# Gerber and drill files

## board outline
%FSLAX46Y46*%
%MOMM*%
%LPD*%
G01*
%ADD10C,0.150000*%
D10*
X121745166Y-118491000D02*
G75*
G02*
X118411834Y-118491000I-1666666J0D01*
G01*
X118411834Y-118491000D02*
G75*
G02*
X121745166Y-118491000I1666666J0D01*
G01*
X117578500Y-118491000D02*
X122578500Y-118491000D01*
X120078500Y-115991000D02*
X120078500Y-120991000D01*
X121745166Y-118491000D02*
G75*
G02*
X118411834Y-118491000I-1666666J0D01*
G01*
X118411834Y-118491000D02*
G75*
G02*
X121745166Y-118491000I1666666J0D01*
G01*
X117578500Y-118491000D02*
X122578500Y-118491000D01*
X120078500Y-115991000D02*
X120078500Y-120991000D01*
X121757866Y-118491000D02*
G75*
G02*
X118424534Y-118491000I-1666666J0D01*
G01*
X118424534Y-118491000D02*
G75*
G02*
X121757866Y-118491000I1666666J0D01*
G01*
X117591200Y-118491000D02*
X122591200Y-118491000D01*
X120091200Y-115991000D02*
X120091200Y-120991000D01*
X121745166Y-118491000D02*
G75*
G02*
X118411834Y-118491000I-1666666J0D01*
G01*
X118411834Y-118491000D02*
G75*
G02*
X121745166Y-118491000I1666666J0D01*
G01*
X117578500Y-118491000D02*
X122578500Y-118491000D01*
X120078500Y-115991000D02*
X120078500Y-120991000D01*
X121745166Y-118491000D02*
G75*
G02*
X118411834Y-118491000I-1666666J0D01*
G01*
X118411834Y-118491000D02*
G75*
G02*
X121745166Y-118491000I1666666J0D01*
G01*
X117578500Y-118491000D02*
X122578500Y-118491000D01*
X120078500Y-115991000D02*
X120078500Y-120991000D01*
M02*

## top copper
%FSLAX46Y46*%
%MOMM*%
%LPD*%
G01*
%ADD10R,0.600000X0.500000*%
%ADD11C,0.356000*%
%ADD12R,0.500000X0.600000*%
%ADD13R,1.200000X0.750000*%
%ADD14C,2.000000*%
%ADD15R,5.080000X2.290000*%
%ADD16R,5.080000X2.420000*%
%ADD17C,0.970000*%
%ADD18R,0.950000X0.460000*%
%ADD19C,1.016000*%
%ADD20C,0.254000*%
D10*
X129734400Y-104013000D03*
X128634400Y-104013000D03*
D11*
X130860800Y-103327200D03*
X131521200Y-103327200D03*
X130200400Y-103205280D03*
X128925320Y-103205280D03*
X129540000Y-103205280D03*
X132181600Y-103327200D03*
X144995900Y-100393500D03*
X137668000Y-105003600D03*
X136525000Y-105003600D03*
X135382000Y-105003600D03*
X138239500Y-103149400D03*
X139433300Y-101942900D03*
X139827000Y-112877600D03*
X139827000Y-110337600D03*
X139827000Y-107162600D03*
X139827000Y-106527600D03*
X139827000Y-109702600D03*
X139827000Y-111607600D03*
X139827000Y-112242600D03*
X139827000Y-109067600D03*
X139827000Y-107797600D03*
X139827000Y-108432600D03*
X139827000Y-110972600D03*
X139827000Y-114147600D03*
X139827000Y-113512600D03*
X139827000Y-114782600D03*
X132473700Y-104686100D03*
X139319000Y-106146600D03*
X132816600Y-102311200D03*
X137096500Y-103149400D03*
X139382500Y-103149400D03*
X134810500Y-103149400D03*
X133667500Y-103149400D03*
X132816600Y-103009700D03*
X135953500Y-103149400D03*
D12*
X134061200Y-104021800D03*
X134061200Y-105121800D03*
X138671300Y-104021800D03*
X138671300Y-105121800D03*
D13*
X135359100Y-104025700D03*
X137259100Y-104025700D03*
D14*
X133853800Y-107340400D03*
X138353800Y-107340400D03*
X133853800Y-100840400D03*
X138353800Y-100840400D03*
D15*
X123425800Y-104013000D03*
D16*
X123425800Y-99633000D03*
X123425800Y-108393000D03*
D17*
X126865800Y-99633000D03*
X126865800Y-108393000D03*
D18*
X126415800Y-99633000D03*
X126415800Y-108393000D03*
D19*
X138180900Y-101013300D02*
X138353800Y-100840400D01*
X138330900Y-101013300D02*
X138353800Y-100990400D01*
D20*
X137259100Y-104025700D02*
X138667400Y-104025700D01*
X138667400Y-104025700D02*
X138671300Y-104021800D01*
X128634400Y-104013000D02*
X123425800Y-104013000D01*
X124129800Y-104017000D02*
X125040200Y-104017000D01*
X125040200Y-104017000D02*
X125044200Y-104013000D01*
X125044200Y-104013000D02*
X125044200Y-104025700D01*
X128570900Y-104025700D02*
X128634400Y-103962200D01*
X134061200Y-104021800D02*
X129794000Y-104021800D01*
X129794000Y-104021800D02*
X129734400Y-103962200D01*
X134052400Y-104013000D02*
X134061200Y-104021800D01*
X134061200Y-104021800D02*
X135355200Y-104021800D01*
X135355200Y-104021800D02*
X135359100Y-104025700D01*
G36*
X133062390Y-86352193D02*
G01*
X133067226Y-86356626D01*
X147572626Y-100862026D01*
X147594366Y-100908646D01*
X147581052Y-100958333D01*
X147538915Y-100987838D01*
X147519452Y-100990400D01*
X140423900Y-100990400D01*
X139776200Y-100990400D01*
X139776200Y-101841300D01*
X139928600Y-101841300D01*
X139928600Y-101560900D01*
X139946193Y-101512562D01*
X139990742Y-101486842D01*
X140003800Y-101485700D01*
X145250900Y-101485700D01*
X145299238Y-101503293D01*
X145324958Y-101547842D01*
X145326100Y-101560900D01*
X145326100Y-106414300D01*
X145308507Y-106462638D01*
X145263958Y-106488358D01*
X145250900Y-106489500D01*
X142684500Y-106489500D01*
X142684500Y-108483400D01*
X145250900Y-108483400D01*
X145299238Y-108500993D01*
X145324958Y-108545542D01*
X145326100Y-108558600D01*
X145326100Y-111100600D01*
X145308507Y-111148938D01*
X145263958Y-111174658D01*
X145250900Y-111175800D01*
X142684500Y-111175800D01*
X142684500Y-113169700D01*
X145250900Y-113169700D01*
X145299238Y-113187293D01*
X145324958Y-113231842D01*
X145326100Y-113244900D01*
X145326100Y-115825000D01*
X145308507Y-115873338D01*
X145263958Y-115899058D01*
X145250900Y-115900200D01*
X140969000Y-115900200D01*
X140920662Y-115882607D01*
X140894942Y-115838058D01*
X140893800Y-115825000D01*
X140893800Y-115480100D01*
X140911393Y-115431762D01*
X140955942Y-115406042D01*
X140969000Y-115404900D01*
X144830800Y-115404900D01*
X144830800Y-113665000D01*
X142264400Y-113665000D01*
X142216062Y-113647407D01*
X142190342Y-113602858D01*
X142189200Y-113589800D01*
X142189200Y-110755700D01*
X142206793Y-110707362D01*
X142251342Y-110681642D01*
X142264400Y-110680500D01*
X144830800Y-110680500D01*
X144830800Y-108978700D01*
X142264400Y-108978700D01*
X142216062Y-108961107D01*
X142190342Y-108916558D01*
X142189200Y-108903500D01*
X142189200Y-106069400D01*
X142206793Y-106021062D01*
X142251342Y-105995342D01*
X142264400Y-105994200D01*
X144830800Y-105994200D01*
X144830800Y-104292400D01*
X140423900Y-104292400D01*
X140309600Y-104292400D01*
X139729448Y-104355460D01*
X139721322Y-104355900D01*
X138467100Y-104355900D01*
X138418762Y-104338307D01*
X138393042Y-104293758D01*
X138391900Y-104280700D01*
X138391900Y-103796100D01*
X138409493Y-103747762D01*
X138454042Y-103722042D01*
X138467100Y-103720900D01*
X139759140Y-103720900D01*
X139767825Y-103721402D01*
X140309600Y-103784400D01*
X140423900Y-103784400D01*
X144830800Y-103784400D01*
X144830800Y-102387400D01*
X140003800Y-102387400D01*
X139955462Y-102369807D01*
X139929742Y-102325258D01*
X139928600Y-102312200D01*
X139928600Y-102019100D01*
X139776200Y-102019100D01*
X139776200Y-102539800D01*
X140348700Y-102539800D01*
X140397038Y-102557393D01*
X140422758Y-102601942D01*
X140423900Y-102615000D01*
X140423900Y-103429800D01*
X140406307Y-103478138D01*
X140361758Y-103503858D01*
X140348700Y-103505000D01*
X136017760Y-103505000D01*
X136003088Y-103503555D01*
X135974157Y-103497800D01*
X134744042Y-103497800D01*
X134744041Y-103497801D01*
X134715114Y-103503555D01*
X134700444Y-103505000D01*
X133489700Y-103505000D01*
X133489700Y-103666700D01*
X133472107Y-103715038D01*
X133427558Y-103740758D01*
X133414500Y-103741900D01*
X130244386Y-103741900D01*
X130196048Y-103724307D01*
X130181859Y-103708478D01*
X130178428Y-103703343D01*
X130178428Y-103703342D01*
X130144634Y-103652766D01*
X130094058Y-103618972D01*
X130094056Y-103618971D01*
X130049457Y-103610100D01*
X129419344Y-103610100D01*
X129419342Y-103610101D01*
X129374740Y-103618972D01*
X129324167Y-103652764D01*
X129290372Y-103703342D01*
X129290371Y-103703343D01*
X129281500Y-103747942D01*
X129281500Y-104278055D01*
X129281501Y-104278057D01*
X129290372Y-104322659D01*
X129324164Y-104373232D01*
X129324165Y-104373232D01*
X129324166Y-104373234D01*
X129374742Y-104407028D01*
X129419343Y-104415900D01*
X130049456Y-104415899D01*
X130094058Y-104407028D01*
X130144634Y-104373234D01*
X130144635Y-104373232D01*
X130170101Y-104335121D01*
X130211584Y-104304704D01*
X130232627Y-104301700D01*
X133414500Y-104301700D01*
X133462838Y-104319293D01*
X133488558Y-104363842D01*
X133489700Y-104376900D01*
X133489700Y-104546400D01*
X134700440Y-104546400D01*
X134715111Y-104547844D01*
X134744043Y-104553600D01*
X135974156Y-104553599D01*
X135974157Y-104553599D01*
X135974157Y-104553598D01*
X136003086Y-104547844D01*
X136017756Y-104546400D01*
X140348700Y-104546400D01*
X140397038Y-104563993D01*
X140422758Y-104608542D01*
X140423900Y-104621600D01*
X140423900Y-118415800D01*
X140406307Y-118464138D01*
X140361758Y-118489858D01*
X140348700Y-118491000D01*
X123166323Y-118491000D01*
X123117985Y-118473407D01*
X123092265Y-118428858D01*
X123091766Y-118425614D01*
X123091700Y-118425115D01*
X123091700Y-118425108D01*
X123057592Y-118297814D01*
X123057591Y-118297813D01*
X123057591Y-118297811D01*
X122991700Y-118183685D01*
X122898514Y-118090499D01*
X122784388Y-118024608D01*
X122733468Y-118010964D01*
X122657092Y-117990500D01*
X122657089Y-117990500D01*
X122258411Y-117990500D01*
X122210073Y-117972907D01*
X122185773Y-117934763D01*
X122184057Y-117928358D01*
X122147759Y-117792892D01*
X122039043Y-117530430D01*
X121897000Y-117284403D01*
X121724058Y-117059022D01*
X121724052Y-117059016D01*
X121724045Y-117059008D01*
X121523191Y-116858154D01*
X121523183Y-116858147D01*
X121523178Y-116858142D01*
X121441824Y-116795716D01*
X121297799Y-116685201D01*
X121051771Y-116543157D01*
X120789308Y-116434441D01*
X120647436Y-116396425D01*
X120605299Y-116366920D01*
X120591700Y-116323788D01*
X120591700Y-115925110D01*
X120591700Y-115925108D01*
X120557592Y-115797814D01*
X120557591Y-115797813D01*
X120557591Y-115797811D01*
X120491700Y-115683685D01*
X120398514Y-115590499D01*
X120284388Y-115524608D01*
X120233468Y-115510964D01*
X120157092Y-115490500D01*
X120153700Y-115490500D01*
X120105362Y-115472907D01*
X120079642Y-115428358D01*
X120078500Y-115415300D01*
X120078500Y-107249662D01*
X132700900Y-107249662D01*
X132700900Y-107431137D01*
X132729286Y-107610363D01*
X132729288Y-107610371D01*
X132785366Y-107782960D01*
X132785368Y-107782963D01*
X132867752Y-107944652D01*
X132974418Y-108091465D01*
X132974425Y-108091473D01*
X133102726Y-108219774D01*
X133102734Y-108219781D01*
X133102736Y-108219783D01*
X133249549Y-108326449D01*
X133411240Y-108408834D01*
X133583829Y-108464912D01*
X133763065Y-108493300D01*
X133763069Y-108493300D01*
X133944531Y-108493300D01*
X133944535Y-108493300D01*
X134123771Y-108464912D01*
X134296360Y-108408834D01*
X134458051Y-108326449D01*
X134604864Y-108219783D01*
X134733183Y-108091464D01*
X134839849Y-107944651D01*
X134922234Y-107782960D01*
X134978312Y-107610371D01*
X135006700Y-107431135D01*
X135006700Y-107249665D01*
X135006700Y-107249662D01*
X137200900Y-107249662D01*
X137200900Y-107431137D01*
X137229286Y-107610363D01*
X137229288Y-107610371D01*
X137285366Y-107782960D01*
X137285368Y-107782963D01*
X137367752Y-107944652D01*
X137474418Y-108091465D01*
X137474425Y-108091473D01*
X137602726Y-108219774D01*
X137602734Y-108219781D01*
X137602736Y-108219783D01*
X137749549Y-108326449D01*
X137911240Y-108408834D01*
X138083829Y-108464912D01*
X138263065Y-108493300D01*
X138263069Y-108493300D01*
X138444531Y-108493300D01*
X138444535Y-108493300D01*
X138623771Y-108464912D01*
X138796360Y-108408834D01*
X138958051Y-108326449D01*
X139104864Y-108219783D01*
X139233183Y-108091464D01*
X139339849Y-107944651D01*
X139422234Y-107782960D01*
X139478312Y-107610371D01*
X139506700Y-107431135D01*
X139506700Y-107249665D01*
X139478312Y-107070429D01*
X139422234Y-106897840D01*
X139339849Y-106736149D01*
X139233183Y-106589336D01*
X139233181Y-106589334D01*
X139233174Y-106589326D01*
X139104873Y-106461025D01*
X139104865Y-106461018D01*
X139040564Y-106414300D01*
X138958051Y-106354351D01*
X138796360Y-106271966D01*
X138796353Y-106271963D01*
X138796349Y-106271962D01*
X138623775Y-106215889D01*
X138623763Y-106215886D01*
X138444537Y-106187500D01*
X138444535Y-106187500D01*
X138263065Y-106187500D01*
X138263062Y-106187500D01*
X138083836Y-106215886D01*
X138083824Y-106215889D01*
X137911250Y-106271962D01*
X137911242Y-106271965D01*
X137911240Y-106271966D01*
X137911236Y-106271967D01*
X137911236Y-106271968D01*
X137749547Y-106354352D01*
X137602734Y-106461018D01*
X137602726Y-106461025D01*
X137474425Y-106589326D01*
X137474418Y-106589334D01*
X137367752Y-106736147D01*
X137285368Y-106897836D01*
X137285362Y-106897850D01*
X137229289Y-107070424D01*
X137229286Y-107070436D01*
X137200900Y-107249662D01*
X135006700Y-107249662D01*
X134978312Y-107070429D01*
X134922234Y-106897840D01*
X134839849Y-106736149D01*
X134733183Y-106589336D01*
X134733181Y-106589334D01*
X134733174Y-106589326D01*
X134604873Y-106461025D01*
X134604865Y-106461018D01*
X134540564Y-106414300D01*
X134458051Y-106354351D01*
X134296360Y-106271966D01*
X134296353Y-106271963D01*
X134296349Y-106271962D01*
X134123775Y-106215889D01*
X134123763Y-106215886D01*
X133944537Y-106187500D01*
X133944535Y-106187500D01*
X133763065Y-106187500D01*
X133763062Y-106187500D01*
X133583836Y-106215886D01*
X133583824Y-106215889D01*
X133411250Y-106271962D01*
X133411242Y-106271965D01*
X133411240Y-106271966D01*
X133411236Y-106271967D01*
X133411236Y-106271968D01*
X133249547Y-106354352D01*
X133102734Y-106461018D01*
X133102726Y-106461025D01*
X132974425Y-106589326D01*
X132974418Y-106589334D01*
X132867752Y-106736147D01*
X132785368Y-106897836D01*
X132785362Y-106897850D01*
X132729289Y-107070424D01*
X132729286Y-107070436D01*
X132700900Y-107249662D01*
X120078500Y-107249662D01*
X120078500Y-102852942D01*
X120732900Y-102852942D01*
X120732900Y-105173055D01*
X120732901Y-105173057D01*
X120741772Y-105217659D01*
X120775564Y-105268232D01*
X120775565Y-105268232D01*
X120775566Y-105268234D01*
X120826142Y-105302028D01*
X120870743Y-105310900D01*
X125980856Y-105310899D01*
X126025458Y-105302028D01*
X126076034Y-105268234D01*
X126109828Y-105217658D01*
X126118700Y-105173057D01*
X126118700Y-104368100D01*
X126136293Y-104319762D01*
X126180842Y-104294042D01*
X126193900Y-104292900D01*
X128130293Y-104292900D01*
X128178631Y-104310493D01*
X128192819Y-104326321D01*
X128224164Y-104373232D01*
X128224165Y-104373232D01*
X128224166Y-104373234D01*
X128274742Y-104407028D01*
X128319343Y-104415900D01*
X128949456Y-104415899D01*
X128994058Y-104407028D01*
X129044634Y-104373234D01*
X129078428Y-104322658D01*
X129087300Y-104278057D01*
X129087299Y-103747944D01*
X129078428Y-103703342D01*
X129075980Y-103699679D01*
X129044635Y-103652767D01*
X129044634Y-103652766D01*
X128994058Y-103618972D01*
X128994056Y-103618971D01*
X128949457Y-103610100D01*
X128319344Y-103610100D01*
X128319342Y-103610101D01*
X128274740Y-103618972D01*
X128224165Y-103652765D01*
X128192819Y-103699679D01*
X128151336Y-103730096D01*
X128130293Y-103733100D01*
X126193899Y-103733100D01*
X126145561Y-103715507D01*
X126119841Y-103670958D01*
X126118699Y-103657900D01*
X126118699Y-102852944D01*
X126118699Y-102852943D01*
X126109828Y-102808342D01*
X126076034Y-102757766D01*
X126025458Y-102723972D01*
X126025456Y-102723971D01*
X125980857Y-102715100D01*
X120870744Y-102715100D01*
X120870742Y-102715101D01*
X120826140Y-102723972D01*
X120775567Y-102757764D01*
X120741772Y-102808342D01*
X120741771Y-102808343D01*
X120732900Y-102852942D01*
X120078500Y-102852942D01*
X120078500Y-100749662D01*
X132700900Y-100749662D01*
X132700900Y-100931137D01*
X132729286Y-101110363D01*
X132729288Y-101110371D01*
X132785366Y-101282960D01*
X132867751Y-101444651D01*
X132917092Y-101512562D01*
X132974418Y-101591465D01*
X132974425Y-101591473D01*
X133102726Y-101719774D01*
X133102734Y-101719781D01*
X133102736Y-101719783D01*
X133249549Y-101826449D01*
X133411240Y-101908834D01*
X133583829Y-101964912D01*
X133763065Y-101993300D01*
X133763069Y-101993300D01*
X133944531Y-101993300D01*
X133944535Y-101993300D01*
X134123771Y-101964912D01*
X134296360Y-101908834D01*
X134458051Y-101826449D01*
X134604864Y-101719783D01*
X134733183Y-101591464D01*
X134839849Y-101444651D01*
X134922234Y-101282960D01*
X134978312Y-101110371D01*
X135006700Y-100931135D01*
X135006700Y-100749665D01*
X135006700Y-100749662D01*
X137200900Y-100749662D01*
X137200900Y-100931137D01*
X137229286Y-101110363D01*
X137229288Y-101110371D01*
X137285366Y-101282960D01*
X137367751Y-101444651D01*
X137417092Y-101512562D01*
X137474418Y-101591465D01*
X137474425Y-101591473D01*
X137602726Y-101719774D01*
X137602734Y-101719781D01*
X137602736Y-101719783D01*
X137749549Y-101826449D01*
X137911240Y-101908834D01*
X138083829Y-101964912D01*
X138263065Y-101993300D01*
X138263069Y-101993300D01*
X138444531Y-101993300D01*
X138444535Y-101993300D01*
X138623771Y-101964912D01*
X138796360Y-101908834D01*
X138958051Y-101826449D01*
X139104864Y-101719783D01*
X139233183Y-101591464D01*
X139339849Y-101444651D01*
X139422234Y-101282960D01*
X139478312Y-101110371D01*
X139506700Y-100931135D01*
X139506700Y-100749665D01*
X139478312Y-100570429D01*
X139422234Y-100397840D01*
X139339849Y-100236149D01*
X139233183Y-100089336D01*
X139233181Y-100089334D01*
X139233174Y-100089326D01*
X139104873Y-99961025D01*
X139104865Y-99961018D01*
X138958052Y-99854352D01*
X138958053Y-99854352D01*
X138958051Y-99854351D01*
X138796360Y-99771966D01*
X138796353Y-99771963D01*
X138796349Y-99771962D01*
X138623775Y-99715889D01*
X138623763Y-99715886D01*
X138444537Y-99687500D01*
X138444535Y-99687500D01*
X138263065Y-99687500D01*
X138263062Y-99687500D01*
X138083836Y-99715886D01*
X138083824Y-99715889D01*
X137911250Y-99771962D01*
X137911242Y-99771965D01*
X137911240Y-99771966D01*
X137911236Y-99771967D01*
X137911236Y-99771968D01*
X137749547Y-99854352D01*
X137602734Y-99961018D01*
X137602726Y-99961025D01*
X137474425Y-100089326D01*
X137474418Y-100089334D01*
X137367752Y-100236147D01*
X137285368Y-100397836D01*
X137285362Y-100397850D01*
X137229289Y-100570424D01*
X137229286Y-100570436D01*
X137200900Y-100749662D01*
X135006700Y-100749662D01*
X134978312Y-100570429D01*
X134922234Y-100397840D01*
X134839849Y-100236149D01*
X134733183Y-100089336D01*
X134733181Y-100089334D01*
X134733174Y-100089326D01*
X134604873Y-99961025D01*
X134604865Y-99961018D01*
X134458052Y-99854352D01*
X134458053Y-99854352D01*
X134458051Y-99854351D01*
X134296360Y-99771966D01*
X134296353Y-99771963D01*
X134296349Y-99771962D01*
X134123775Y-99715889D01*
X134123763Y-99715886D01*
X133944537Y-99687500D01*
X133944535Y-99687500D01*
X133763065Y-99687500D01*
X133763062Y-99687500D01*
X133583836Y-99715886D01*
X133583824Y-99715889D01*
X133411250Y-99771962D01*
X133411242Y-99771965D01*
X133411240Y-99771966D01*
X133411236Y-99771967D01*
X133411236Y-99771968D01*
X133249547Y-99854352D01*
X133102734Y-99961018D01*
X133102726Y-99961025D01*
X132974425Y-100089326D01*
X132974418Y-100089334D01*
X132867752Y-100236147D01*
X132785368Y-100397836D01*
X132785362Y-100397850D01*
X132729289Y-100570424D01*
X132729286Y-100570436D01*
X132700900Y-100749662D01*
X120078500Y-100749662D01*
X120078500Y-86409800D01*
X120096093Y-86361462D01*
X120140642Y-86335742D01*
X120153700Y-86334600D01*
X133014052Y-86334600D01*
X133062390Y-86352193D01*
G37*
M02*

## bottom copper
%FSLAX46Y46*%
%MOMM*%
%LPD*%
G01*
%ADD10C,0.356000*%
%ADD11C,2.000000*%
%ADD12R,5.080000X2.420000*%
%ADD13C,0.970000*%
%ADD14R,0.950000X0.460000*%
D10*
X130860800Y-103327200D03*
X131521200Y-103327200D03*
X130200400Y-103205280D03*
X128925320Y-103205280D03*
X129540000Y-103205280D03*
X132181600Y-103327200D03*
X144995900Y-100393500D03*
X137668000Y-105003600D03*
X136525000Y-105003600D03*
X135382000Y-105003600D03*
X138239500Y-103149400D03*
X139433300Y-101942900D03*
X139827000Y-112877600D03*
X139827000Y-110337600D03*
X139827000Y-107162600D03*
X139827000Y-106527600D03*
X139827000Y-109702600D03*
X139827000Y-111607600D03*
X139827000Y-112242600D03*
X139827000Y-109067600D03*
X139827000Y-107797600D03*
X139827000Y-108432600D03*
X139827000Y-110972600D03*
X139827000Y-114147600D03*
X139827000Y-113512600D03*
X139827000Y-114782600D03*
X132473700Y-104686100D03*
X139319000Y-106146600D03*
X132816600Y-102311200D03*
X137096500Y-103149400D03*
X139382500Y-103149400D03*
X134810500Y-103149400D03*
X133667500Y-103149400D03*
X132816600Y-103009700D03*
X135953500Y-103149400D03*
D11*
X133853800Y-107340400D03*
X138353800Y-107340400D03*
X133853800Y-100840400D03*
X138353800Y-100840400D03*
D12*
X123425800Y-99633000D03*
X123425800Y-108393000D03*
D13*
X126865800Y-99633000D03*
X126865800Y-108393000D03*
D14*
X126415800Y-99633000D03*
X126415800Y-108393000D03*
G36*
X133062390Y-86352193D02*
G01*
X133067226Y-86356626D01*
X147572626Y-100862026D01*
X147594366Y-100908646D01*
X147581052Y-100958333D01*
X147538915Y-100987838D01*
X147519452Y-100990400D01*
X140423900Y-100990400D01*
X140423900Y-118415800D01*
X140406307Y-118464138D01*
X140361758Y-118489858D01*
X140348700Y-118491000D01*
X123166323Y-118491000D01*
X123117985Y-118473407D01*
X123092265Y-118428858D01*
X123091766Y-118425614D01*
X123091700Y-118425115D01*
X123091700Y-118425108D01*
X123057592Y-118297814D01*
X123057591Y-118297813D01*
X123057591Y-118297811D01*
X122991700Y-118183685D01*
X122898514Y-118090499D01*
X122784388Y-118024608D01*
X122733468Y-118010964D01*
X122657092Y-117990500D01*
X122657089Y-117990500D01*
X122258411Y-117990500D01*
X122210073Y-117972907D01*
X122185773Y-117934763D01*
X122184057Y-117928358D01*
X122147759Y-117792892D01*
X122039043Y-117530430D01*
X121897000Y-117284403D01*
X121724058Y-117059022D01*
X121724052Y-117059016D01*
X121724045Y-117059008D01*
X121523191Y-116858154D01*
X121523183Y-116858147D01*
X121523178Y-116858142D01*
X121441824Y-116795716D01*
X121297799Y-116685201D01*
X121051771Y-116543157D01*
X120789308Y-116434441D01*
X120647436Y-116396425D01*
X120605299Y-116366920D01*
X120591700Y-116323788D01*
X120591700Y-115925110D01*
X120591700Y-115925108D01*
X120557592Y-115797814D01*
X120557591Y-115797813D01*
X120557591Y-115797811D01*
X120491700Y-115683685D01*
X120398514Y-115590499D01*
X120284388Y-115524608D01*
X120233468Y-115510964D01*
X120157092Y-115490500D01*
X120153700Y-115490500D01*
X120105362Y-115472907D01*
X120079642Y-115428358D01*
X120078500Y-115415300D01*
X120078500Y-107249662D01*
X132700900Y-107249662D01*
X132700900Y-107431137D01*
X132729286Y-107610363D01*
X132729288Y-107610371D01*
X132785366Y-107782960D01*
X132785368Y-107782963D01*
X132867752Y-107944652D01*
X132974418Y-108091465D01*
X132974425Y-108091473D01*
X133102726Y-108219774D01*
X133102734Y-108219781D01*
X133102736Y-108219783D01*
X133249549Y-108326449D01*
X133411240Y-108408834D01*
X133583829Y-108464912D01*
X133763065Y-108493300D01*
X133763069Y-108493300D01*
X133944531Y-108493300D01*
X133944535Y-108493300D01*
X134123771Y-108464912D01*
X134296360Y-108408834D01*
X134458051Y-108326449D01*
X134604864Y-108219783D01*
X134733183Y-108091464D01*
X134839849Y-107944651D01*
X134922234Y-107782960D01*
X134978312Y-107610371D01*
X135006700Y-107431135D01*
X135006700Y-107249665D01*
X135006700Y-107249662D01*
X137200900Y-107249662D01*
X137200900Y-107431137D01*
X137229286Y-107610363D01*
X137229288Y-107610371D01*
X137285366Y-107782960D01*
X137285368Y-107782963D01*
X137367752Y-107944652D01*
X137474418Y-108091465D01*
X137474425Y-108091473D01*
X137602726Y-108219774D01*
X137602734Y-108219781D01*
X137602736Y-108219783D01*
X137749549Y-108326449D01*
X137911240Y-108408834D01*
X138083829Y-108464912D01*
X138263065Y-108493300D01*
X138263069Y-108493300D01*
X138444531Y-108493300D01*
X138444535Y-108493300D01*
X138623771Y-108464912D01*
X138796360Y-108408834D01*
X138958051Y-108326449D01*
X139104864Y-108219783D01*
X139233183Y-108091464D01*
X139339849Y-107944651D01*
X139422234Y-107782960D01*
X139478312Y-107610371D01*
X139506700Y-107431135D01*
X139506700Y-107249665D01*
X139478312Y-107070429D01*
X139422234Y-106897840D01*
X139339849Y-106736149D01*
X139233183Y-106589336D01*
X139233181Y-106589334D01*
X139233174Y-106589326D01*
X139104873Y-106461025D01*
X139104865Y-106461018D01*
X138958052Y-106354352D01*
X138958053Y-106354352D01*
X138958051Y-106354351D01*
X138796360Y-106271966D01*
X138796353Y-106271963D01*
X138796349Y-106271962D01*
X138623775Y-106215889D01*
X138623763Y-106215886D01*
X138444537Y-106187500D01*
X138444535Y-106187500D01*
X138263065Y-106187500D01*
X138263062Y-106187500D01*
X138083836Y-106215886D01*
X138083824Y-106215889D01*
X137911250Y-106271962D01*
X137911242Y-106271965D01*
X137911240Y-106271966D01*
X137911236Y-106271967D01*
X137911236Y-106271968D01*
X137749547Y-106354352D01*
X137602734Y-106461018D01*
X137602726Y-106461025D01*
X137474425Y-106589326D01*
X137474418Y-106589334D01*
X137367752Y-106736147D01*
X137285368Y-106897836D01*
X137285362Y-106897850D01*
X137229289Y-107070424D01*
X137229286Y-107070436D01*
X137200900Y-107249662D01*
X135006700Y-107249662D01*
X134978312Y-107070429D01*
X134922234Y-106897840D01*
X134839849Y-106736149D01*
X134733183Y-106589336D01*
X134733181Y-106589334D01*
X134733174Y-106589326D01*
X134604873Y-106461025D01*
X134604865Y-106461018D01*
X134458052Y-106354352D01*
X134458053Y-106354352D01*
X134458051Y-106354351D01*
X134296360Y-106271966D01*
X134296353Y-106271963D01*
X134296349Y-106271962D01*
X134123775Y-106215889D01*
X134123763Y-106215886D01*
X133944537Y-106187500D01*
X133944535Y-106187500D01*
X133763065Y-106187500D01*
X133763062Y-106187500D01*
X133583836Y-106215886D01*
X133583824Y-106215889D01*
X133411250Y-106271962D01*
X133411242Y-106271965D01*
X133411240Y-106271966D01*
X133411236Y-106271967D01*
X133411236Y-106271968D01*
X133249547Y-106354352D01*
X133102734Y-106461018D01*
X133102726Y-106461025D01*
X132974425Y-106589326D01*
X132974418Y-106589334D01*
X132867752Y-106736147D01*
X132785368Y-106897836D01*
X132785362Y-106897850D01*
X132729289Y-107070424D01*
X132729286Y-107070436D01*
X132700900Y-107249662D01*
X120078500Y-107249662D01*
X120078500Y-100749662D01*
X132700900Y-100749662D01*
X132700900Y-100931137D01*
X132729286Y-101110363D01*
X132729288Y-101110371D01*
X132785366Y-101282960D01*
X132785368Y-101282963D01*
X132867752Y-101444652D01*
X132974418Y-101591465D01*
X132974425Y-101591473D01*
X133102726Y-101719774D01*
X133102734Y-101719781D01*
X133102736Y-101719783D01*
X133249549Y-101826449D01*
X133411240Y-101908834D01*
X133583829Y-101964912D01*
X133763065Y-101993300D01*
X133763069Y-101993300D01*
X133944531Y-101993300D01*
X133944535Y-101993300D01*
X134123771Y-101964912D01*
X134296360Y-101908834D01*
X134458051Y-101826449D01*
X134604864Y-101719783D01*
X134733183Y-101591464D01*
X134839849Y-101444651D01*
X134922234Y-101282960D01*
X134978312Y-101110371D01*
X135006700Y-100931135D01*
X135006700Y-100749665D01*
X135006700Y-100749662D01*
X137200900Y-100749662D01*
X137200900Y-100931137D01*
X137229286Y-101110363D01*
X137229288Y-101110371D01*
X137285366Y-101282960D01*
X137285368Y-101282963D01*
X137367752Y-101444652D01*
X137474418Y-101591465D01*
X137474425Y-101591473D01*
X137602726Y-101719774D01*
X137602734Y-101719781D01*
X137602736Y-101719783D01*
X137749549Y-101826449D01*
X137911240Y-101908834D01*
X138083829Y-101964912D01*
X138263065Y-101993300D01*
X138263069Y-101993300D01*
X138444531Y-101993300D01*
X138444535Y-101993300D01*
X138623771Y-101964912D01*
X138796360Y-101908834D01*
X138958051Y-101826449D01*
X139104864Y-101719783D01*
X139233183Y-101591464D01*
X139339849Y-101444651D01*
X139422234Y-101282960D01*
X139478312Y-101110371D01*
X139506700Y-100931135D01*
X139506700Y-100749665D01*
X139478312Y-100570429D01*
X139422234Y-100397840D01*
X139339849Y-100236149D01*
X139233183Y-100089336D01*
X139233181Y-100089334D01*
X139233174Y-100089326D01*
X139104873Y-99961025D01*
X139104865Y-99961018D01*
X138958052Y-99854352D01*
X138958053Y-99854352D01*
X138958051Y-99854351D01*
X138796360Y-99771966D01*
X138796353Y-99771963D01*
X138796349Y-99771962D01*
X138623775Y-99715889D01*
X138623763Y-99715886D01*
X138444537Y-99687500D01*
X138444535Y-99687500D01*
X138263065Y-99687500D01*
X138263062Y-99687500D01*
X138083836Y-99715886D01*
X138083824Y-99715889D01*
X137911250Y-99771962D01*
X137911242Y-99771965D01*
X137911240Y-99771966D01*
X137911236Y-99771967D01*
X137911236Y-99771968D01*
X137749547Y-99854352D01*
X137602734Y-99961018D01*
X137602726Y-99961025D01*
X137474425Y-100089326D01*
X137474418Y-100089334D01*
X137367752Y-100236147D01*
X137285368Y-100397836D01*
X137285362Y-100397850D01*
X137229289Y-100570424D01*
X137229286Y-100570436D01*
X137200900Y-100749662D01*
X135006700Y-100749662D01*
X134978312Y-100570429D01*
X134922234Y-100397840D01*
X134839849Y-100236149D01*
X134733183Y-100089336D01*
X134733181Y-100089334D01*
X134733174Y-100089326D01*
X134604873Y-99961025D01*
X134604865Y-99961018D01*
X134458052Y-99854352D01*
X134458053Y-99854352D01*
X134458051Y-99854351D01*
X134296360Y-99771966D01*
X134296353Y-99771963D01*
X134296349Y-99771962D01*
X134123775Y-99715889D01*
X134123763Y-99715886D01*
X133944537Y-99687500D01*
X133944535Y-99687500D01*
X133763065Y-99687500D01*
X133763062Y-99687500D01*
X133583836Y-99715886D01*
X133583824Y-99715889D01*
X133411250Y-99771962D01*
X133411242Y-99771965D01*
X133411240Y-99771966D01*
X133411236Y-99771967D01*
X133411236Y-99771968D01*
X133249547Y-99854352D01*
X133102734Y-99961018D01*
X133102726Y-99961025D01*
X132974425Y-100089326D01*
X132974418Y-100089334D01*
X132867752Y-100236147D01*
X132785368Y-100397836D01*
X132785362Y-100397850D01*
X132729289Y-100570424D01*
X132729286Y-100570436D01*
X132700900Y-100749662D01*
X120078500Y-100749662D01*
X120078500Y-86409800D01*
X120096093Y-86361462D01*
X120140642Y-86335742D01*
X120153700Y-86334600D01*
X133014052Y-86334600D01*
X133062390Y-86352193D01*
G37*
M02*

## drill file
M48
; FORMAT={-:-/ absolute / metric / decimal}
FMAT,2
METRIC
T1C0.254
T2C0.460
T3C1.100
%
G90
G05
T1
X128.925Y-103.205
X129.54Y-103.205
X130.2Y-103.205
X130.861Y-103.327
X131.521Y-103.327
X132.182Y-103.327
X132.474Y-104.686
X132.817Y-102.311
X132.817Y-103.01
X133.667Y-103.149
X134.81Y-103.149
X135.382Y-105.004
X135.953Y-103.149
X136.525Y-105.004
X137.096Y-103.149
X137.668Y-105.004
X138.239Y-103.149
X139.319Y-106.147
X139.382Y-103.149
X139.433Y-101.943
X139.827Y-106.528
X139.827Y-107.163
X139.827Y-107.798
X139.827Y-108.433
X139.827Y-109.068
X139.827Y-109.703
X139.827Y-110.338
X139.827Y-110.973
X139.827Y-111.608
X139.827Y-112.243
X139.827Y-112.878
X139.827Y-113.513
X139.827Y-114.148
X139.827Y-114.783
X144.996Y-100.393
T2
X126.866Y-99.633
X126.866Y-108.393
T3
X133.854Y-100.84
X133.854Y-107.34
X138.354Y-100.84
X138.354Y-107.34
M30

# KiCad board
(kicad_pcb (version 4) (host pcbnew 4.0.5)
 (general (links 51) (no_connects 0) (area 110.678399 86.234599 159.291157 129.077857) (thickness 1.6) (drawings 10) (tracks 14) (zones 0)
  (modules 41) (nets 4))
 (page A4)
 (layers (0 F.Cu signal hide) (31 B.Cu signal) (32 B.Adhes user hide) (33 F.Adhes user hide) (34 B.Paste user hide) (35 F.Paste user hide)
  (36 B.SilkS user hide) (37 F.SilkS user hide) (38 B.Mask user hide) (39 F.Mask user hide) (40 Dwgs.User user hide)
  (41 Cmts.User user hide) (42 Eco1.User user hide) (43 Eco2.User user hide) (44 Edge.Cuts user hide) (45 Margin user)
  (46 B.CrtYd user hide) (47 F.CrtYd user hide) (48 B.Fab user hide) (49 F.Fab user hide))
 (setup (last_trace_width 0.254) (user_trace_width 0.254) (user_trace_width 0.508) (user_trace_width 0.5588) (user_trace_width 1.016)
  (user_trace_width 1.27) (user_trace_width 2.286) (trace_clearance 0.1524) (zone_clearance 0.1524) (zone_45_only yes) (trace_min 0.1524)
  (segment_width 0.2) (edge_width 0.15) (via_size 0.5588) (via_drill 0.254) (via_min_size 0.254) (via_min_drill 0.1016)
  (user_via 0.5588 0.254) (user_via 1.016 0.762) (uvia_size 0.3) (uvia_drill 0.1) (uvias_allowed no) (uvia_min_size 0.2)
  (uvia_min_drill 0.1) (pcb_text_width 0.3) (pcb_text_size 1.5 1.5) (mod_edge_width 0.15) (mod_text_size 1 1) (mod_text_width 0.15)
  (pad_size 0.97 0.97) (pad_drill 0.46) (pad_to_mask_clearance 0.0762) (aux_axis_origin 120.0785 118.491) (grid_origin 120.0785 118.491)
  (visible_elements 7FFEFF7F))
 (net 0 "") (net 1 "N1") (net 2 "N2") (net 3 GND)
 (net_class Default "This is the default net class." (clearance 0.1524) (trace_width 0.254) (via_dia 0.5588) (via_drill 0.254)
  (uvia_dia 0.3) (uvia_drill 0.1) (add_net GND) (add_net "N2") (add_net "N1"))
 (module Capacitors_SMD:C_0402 (layer F.Cu) (at 129.1844 104.013 180)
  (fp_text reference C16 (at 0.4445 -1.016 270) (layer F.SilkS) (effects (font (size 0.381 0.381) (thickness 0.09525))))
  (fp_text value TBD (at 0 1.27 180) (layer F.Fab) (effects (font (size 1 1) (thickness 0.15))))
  (pad 1 smd rect (at -0.55 0 180) (size 0.6 0.5) (layers F.Cu F.Paste F.Mask) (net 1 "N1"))
  (pad 2 smd rect (at 0.55 0 180) (size 0.6 0.5) (layers F.Cu F.Paste F.Mask) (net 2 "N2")))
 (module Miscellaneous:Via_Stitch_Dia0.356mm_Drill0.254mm (layer F.Cu) (at 130.8608 103.3272)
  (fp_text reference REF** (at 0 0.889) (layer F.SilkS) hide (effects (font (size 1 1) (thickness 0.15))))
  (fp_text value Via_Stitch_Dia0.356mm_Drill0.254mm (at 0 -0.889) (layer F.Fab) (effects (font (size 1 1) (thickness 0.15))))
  (pad 1 thru_hole circle (at 0 0) (size 0.356 0.356) (drill 0.254) (layers *.Cu) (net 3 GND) (zone_connect 2)))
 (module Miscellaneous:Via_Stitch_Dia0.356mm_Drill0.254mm (layer B.Cu) (at 131.5212 103.3272)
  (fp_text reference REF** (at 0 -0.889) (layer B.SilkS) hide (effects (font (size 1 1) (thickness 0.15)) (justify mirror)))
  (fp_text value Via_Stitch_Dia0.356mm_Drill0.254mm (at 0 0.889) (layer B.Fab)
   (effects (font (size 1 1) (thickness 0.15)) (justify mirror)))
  (pad 1 thru_hole circle (at 0 0) (size 0.356 0.356) (drill 0.254) (layers *.Cu) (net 3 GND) (zone_connect 2)))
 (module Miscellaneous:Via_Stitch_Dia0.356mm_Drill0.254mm (layer B.Cu) (at 130.2004 103.20528)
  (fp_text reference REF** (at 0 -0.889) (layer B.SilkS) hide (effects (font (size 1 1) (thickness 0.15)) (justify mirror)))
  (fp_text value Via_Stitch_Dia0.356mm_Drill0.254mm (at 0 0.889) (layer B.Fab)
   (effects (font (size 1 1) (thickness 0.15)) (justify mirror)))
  (pad 1 thru_hole circle (at 0 0) (size 0.356 0.356) (drill 0.254) (layers *.Cu) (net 3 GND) (zone_connect 2)))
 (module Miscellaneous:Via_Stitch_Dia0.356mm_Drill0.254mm (layer B.Cu) (at 128.92532 103.20528)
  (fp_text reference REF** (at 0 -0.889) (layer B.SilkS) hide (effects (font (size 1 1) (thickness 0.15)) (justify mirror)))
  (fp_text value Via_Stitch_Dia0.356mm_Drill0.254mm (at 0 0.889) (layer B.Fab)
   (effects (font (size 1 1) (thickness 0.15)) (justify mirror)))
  (pad 1 thru_hole circle (at 0 0) (size 0.356 0.356) (drill 0.254) (layers *.Cu) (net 3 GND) (zone_connect 2)))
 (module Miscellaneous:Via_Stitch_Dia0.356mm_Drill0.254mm (layer B.Cu) (at 129.54 103.20528)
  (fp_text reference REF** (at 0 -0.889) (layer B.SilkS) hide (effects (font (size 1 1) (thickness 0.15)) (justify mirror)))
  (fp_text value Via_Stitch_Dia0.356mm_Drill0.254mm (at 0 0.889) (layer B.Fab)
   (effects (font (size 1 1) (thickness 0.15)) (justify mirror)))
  (pad 1 thru_hole circle (at 0 0) (size 0.356 0.356) (drill 0.254) (layers *.Cu) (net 3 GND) (zone_connect 2)))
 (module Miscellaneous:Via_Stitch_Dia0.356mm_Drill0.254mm (layer B.Cu) (at 132.1816 103.3272)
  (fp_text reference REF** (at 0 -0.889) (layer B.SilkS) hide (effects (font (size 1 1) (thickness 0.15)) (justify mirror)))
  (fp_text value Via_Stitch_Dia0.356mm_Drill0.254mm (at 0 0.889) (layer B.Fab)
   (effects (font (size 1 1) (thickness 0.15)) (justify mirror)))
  (pad 1 thru_hole circle (at 0 0) (size 0.356 0.356) (drill 0.254) (layers *.Cu) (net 3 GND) (zone_connect 2)))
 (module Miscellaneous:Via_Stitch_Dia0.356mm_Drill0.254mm (layer B.Cu) (at 144.9959 100.3935)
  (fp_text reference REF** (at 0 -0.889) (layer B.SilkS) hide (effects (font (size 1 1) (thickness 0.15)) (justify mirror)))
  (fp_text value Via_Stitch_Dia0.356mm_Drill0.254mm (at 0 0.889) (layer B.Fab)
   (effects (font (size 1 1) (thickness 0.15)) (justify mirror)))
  (pad 1 thru_hole circle (at 0 0) (size 0.356 0.356) (drill 0.254) (layers *.Cu) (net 3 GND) (zone_connect 2)))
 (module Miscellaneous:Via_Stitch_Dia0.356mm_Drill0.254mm (layer B.Cu) (at 137.668 105.0036)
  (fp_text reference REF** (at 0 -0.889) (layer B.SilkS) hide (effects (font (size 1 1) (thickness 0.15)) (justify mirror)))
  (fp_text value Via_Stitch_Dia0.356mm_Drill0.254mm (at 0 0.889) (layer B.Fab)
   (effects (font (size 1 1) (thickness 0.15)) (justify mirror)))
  (pad 1 thru_hole circle (at 0 0) (size 0.356 0.356) (drill 0.254) (layers *.Cu) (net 3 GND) (zone_connect 2)))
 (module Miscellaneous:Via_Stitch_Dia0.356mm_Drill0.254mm (layer B.Cu) (at 136.525 105.0036)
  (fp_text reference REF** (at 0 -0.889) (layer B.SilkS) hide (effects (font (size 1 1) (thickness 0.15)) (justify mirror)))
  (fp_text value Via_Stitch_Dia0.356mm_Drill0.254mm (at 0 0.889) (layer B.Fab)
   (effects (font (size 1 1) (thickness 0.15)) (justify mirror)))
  (pad 1 thru_hole circle (at 0 0) (size 0.356 0.356) (drill 0.254) (layers *.Cu) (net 3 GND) (zone_connect 2)))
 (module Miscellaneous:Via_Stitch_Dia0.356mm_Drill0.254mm (layer B.Cu) (at 135.382 105.0036)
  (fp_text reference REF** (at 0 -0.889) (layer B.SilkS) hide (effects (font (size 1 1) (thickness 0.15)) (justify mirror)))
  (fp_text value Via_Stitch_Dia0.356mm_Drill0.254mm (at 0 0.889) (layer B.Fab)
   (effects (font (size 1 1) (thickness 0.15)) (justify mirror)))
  (pad 1 thru_hole circle (at 0 0) (size 0.356 0.356) (drill 0.254) (layers *.Cu) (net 3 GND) (zone_connect 2)))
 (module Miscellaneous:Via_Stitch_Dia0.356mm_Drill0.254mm (layer B.Cu) (at 138.2395 103.1494)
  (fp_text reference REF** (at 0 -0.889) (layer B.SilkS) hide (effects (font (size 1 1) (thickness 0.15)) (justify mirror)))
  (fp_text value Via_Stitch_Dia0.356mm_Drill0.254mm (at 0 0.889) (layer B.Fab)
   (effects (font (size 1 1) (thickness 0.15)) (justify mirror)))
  (pad 1 thru_hole circle (at 0 0) (size 0.356 0.356) (drill 0.254) (layers *.Cu) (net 3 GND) (zone_connect 2)))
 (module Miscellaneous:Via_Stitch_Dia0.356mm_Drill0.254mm (layer B.Cu) (at 139.4333 101.9429)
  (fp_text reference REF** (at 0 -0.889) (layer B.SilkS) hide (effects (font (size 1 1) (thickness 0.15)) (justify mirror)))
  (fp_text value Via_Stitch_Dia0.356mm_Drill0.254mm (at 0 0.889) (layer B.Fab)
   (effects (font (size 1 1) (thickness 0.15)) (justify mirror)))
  (pad 1 thru_hole circle (at 0 0) (size 0.356 0.356) (drill 0.254) (layers *.Cu) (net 3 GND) (zone_connect 2)))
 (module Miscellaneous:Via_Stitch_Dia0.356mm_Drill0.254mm (layer B.Cu) (at 139.827 112.8776 90)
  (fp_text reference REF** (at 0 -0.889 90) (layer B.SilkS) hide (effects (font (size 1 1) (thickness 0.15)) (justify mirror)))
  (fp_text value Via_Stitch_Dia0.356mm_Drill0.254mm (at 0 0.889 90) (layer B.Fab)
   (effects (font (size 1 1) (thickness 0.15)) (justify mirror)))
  (pad 1 thru_hole circle (at 0 0 90) (size 0.356 0.356) (drill 0.254) (layers *.Cu) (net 3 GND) (zone_connect 2)))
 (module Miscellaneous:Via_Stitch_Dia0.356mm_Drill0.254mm (layer B.Cu) (at 139.827 110.3376 90)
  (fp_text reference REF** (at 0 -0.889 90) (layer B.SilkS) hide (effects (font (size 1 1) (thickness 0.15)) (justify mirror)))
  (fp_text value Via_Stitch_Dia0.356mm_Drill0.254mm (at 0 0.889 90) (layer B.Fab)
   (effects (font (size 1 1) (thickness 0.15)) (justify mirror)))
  (pad 1 thru_hole circle (at 0 0 90) (size 0.356 0.356) (drill 0.254) (layers *.Cu) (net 3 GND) (zone_connect 2)))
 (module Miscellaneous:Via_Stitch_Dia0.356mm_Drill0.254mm (layer B.Cu) (at 139.827 107.1626 90)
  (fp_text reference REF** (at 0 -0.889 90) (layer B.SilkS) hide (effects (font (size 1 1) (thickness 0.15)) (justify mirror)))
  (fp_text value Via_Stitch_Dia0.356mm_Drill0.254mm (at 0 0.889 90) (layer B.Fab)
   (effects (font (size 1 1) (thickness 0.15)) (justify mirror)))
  (pad 1 thru_hole circle (at 0 0 90) (size 0.356 0.356) (drill 0.254) (layers *.Cu) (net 3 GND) (zone_connect 2)))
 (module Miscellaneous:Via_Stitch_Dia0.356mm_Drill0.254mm (layer B.Cu) (at 139.827 106.5276 90)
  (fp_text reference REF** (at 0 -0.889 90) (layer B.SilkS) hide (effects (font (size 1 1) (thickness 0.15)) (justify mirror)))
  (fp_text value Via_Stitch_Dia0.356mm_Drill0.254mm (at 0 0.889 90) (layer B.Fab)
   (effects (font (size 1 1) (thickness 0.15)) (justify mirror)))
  (pad 1 thru_hole circle (at 0 0 90) (size 0.356 0.356) (drill 0.254) (layers *.Cu) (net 3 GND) (zone_connect 2)))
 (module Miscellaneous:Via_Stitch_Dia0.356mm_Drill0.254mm (layer B.Cu) (at 139.827 109.7026 90)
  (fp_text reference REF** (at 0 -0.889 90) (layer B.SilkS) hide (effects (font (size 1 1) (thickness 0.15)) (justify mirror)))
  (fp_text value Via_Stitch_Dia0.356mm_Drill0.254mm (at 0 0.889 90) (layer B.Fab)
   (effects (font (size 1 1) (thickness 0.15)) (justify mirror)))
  (pad 1 thru_hole circle (at 0 0 90) (size 0.356 0.356) (drill 0.254) (layers *.Cu) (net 3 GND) (zone_connect 2)))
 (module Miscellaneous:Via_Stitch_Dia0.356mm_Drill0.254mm (layer B.Cu) (at 139.827 111.6076 90)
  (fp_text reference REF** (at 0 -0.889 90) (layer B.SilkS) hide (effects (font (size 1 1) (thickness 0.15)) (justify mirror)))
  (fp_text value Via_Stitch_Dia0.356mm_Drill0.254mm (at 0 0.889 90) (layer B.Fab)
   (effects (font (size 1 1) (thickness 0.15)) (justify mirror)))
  (pad 1 thru_hole circle (at 0 0 90) (size 0.356 0.356) (drill 0.254) (layers *.Cu) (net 3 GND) (zone_connect 2)))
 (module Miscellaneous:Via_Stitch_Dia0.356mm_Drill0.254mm (layer B.Cu) (at 139.827 112.2426 90)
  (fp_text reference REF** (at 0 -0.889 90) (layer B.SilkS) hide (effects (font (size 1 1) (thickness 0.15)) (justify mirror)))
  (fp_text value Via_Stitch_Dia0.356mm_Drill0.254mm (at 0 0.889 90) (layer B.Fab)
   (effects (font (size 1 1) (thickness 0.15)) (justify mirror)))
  (pad 1 thru_hole circle (at 0 0 90) (size 0.356 0.356) (drill 0.254) (layers *.Cu) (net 3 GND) (zone_connect 2)))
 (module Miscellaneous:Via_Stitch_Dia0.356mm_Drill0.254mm (layer B.Cu) (at 139.827 109.0676 90)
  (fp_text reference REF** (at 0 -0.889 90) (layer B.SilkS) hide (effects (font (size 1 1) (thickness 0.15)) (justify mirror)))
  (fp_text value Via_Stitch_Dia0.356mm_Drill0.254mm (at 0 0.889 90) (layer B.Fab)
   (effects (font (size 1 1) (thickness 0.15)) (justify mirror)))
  (pad 1 thru_hole circle (at 0 0 90) (size 0.356 0.356) (drill 0.254) (layers *.Cu) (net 3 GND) (zone_connect 2)))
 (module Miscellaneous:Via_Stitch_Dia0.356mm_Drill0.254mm (layer B.Cu) (at 139.827 107.7976 90)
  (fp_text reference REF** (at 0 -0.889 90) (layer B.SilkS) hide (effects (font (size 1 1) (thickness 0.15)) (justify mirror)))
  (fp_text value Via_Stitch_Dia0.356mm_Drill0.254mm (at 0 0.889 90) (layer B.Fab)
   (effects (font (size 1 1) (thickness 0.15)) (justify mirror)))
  (pad 1 thru_hole circle (at 0 0 90) (size 0.356 0.356) (drill 0.254) (layers *.Cu) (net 3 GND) (zone_connect 2)))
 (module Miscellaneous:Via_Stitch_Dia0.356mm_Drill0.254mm (layer B.Cu) (at 139.827 108.4326 90)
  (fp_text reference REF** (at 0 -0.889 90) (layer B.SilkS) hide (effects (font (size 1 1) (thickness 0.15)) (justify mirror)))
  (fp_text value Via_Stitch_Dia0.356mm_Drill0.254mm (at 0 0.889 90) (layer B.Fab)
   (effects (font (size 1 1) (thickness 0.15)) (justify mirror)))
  (pad 1 thru_hole circle (at 0 0 90) (size 0.356 0.356) (drill 0.254) (layers *.Cu) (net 3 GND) (zone_connect 2)))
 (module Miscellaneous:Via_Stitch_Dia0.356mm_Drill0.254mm (layer B.Cu) (at 139.827 110.9726 90)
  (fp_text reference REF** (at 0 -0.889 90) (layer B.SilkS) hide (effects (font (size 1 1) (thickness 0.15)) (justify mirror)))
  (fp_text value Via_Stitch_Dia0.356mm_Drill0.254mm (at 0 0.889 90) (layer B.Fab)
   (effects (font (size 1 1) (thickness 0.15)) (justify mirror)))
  (pad 1 thru_hole circle (at 0 0 90) (size 0.356 0.356) (drill 0.254) (layers *.Cu) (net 3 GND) (zone_connect 2)))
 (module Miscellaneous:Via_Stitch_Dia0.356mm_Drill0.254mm (layer B.Cu) (at 139.827 114.1476 90)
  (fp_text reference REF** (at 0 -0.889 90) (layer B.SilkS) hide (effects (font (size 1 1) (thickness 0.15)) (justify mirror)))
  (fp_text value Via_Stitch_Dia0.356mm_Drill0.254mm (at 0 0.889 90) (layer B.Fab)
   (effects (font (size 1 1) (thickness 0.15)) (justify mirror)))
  (pad 1 thru_hole circle (at 0 0 90) (size 0.356 0.356) (drill 0.254) (layers *.Cu) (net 3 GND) (zone_connect 2)))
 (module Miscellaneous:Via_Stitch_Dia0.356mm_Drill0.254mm (layer B.Cu) (at 139.827 113.5126 90)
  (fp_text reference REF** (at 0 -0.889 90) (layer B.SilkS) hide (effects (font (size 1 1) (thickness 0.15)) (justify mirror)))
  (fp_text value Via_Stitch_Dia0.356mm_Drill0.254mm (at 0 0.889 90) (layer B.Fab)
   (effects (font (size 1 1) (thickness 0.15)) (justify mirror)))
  (pad 1 thru_hole circle (at 0 0 90) (size 0.356 0.356) (drill 0.254) (layers *.Cu) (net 3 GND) (zone_connect 2)))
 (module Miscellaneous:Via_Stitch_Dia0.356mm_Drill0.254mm (layer B.Cu) (at 139.827 114.7826 90)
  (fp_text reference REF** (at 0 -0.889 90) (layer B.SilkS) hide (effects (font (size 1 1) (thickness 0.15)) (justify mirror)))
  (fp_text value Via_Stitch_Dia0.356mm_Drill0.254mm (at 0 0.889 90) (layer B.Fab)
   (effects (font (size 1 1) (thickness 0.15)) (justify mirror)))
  (pad 1 thru_hole circle (at 0 0 90) (size 0.356 0.356) (drill 0.254) (layers *.Cu) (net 3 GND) (zone_connect 2)))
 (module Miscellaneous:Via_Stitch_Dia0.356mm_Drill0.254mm (layer B.Cu) (at 132.4737 104.6861 90)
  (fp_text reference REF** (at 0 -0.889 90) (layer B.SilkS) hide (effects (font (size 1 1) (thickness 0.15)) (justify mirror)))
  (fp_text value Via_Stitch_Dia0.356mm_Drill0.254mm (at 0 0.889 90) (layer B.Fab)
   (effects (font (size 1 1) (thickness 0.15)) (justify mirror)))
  (pad 1 thru_hole circle (at 0 0 90) (size 0.356 0.356) (drill 0.254) (layers *.Cu) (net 3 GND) (zone_connect 2)))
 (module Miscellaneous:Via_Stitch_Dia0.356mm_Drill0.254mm (layer B.Cu) (at 139.319 106.1466)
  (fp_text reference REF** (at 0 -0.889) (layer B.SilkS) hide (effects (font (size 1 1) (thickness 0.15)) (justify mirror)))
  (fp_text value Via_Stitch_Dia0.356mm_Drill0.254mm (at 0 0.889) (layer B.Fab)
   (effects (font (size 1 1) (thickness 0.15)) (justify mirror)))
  (pad 1 thru_hole circle (at 0 0) (size 0.356 0.356) (drill 0.254) (layers *.Cu) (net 3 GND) (zone_connect 2)))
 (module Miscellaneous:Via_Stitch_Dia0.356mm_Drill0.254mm (layer B.Cu) (at 132.8166 102.3112)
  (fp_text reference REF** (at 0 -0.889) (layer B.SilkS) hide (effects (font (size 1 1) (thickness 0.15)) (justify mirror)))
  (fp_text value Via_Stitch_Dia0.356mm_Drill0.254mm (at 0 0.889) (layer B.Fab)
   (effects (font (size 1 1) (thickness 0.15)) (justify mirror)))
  (pad 1 thru_hole circle (at 0 0) (size 0.356 0.356) (drill 0.254) (layers *.Cu) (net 3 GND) (zone_connect 2)))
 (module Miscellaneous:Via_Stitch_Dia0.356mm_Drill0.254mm (layer B.Cu) (at 137.0965 103.1494)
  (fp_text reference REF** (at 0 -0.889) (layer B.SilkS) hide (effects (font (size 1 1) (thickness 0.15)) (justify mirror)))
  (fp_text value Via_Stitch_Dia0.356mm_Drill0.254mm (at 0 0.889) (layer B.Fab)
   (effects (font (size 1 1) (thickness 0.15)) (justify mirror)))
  (pad 1 thru_hole circle (at 0 0) (size 0.356 0.356) (drill 0.254) (layers *.Cu) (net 3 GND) (zone_connect 2)))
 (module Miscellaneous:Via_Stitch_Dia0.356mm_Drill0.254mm (layer B.Cu) (at 139.3825 103.1494)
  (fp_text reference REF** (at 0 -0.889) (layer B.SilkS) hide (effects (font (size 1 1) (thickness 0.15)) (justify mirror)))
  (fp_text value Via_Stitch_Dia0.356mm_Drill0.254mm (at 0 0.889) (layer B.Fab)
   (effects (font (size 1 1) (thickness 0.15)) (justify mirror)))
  (pad 1 thru_hole circle (at 0 0) (size 0.356 0.356) (drill 0.254) (layers *.Cu) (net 3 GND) (zone_connect 2)))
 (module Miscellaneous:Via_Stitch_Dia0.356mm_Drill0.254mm (layer F.Cu) (at 134.8105 103.1494)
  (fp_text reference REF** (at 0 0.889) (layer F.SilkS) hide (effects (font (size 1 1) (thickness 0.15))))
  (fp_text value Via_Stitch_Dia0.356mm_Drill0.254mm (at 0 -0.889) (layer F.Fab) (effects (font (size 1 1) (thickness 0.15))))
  (pad 1 thru_hole circle (at 0 0) (size 0.356 0.356) (drill 0.254) (layers *.Cu) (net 3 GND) (zone_connect 2)))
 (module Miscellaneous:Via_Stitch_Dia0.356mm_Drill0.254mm (layer B.Cu) (at 133.6675 103.1494)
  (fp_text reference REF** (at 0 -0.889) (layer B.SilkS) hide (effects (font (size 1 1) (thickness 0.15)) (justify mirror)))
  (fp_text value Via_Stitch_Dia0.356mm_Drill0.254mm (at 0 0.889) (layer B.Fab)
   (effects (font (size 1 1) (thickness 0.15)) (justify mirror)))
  (pad 1 thru_hole circle (at 0 0) (size 0.356 0.356) (drill 0.254) (layers *.Cu) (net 3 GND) (zone_connect 2)))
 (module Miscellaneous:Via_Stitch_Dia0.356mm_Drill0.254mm (layer B.Cu) (at 132.8166 103.0097)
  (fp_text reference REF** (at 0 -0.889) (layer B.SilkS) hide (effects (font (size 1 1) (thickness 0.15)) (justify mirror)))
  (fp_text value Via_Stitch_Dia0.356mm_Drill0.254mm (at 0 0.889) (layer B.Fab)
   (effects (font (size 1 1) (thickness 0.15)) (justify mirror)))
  (pad 1 thru_hole circle (at 0 0) (size 0.356 0.356) (drill 0.254) (layers *.Cu) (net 3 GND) (zone_connect 2)))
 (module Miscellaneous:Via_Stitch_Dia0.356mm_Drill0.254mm (layer B.Cu) (at 135.9535 103.1494)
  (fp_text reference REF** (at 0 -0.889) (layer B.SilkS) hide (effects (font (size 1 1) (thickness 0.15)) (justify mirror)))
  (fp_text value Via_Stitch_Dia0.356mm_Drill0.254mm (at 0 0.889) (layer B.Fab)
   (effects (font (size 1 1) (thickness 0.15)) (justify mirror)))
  (pad 1 thru_hole circle (at 0 0) (size 0.356 0.356) (drill 0.254) (layers *.Cu) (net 3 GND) (zone_connect 2)))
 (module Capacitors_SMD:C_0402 (layer F.Cu) (at 134.0612 104.5718 270)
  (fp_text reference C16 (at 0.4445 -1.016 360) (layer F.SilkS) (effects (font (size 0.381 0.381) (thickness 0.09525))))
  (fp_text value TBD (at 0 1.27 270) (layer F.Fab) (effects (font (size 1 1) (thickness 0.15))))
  (pad 1 smd rect (at -0.55 0 270) (size 0.6 0.5) (layers F.Cu F.Paste F.Mask) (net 1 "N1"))
  (pad 2 smd rect (at 0.55 0 270) (size 0.6 0.5) (layers F.Cu F.Paste F.Mask) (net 3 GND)))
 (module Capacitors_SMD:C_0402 (layer F.Cu) (at 138.6713 104.5718 270)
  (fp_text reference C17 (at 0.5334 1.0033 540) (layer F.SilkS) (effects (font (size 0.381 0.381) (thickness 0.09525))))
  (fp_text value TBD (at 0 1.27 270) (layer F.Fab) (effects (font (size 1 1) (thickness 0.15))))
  (pad 1 smd rect (at -0.55 0 270) (size 0.6 0.5) (layers F.Cu F.Paste F.Mask) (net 3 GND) (zone_connect 2))
  (pad 2 smd rect (at 0.55 0 270) (size 0.6 0.5) (layers F.Cu F.Paste F.Mask) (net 3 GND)))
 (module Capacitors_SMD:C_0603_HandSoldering (layer F.Cu) (at 136.3091 104.0257)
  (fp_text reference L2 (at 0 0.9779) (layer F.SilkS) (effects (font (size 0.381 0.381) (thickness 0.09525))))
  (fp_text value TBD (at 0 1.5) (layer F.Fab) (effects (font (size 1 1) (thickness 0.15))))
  (pad 1 smd rect (at -0.95 0) (size 1.2 0.75) (layers F.Cu F.Paste F.Mask) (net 1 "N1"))
  (pad 2 smd rect (at 0.95 0) (size 1.2 0.75) (layers F.Cu F.Paste F.Mask) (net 3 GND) (zone_connect 2)))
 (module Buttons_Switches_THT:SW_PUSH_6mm (layer B.Cu) (at 138.3538 107.3404 90)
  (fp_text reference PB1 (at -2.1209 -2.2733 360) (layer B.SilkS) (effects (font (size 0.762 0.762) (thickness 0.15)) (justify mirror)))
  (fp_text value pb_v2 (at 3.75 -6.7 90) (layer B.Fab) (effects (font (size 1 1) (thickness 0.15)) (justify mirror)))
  (pad 2 thru_hole circle (at 0 -4.5) (size 2 2) (drill 1.1) (layers *.Cu *.Mask))
  (pad 1 thru_hole circle (at 0 0) (size 2 2) (drill 1.1) (layers *.Cu *.Mask))
  (pad 2 thru_hole circle (at 6.5 -4.5) (size 2 2) (drill 1.1) (layers *.Cu *.Mask))
  (pad 1 thru_hole circle (at 6.5 0) (size 2 2) (drill 1.1) (layers *.Cu *.Mask)))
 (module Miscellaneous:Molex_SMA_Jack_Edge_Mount (layer F.Cu) (at 125.1458 104.013)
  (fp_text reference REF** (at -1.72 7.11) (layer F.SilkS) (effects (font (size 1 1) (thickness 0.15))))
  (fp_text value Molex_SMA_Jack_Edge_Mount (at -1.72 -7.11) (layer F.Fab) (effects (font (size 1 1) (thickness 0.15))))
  (pad 1 smd rect (at -1.72 0) (size 5.08 2.29) (layers F.Cu F.Paste F.Mask) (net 2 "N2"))
  (pad 2 smd rect (at -1.72 -4.38) (size 5.08 2.42) (layers F.Cu F.Paste F.Mask) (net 3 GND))
  (pad 2 smd rect (at -1.72 4.38) (size 5.08 2.42) (layers F.Cu F.Paste F.Mask) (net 3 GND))
  (pad 2 smd rect (at -1.72 -4.38) (size 5.08 2.42) (layers B.Cu B.Paste B.Mask) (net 3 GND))
  (pad 2 smd rect (at -1.72 4.38) (size 5.08 2.42) (layers B.Cu B.Paste B.Mask) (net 3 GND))
  (pad 2 thru_hole circle (at 1.72 -4.38) (size 0.97 0.97) (drill 0.46) (layers *.Cu) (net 3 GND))
  (pad 2 thru_hole circle (at 1.72 4.38) (size 0.97 0.97) (drill 0.46) (layers *.Cu) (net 3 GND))
  (pad 2 smd rect (at 1.27 -4.38) (size 0.95 0.46) (layers F.Cu) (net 3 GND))
  (pad 2 smd rect (at 1.27 4.38) (size 0.95 0.46) (layers F.Cu) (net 3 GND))
  (pad 2 smd rect (at 1.27 -4.38) (size 0.95 0.46) (layers B.Cu) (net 3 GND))
  (pad 2 smd rect (at 1.27 4.38) (size 0.95 0.46) (layers B.Cu) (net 3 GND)))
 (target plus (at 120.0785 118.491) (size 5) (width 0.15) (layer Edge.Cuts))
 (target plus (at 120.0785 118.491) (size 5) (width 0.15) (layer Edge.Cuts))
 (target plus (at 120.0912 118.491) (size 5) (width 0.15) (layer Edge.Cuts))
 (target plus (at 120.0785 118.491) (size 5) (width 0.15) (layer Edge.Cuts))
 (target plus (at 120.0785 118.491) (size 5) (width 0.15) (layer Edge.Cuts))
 (segment (start 138.1809 101.0133) (end 138.3538 100.8404) (width 1.016) (layer F.Cu) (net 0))
 (segment (start 138.3309 101.0133) (end 138.3538 100.9904) (width 1.016) (layer F.Cu) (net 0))
 (segment (start 137.2591 104.0257) (end 138.6674 104.0257) (width 0.254) (layer F.Cu) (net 3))
 (segment (start 138.6674 104.0257) (end 138.6713 104.0218) (width 0.254) (layer F.Cu) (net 3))
 (segment (start 128.6344 104.013) (end 123.4258 104.013) (width 0.254) (layer F.Cu) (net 2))
 (segment (start 124.1298 104.017) (end 125.0402 104.017) (width 0.254) (layer F.Cu) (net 2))
 (segment (start 125.0402 104.017) (end 125.0442 104.013) (width 0.254) (layer F.Cu) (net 2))
 (segment (start 125.0442 104.013) (end 125.0442 104.0257) (width 0.254) (layer F.Cu) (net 2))
 (segment (start 128.5709 104.0257) (end 128.6344 103.9622) (width 0.254) (layer F.Cu) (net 2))
 (segment (start 134.0612 104.0218) (end 129.794 104.0218) (width 0.254) (layer F.Cu) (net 1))
 (segment (start 129.794 104.0218) (end 129.7344 103.9622) (width 0.254) (layer F.Cu) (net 1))
 (segment (start 134.0524 104.013) (end 134.0612 104.0218) (width 0.254) (layer F.Cu) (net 1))
 (segment (start 134.0612 104.0218) (end 135.3552 104.0218) (width 0.254) (layer F.Cu) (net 1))
 (segment (start 135.3552 104.0218) (end 135.3591 104.0257) (width 0.254) (layer F.Cu) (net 1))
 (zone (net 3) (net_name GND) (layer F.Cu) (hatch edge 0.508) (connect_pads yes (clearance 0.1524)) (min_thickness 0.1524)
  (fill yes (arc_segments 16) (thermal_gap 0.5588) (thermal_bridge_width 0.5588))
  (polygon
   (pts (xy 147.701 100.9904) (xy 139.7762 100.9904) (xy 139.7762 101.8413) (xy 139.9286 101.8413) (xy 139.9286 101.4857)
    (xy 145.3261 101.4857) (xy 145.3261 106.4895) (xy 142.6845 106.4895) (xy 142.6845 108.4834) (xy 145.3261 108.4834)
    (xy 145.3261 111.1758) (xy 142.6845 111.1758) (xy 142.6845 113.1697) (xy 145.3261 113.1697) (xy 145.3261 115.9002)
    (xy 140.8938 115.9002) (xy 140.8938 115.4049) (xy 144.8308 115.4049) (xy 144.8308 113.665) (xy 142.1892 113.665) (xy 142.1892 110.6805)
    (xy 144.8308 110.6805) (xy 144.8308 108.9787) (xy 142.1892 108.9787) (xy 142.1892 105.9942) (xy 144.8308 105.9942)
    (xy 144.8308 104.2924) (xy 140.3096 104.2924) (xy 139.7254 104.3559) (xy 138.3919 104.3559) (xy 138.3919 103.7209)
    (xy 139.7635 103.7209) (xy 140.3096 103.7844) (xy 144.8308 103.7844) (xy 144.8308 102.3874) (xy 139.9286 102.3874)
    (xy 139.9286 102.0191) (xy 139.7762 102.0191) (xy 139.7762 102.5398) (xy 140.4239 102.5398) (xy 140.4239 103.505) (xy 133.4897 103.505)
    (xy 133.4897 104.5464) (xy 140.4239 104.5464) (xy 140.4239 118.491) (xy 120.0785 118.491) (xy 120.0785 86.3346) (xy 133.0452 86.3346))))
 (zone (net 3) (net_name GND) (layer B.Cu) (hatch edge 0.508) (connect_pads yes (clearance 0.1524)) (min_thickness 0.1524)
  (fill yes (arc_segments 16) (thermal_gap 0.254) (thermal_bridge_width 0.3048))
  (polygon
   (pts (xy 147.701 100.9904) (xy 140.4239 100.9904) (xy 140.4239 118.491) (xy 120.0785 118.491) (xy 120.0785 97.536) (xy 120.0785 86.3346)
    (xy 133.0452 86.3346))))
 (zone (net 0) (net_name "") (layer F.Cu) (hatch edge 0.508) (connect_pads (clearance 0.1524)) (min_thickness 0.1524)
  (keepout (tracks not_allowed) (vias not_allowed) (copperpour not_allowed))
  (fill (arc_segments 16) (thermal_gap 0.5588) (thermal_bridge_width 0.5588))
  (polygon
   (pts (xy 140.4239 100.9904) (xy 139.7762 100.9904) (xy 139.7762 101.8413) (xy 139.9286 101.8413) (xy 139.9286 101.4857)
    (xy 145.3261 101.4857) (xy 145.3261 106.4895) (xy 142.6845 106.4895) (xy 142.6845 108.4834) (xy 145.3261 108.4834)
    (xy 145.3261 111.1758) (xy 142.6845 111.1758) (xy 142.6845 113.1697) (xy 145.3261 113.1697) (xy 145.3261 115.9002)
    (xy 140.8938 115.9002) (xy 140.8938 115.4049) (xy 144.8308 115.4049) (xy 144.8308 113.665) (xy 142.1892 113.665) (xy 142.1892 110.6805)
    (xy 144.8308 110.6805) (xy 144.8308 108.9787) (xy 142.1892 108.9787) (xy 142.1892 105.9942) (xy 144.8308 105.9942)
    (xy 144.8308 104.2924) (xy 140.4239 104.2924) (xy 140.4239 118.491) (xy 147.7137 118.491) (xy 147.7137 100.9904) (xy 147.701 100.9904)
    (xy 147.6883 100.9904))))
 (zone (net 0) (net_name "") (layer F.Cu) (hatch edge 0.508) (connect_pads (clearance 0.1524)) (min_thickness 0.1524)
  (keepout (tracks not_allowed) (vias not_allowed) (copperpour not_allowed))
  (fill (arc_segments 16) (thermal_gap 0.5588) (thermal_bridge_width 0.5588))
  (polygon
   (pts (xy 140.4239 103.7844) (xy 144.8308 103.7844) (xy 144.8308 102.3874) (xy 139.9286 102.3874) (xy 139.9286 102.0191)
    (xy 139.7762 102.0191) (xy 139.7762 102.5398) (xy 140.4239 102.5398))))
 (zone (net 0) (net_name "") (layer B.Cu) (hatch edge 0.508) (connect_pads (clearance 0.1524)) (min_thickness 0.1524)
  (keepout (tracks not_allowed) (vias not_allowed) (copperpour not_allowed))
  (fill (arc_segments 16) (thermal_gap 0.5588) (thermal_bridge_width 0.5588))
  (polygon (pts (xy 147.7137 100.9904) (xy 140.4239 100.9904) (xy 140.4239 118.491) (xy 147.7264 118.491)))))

